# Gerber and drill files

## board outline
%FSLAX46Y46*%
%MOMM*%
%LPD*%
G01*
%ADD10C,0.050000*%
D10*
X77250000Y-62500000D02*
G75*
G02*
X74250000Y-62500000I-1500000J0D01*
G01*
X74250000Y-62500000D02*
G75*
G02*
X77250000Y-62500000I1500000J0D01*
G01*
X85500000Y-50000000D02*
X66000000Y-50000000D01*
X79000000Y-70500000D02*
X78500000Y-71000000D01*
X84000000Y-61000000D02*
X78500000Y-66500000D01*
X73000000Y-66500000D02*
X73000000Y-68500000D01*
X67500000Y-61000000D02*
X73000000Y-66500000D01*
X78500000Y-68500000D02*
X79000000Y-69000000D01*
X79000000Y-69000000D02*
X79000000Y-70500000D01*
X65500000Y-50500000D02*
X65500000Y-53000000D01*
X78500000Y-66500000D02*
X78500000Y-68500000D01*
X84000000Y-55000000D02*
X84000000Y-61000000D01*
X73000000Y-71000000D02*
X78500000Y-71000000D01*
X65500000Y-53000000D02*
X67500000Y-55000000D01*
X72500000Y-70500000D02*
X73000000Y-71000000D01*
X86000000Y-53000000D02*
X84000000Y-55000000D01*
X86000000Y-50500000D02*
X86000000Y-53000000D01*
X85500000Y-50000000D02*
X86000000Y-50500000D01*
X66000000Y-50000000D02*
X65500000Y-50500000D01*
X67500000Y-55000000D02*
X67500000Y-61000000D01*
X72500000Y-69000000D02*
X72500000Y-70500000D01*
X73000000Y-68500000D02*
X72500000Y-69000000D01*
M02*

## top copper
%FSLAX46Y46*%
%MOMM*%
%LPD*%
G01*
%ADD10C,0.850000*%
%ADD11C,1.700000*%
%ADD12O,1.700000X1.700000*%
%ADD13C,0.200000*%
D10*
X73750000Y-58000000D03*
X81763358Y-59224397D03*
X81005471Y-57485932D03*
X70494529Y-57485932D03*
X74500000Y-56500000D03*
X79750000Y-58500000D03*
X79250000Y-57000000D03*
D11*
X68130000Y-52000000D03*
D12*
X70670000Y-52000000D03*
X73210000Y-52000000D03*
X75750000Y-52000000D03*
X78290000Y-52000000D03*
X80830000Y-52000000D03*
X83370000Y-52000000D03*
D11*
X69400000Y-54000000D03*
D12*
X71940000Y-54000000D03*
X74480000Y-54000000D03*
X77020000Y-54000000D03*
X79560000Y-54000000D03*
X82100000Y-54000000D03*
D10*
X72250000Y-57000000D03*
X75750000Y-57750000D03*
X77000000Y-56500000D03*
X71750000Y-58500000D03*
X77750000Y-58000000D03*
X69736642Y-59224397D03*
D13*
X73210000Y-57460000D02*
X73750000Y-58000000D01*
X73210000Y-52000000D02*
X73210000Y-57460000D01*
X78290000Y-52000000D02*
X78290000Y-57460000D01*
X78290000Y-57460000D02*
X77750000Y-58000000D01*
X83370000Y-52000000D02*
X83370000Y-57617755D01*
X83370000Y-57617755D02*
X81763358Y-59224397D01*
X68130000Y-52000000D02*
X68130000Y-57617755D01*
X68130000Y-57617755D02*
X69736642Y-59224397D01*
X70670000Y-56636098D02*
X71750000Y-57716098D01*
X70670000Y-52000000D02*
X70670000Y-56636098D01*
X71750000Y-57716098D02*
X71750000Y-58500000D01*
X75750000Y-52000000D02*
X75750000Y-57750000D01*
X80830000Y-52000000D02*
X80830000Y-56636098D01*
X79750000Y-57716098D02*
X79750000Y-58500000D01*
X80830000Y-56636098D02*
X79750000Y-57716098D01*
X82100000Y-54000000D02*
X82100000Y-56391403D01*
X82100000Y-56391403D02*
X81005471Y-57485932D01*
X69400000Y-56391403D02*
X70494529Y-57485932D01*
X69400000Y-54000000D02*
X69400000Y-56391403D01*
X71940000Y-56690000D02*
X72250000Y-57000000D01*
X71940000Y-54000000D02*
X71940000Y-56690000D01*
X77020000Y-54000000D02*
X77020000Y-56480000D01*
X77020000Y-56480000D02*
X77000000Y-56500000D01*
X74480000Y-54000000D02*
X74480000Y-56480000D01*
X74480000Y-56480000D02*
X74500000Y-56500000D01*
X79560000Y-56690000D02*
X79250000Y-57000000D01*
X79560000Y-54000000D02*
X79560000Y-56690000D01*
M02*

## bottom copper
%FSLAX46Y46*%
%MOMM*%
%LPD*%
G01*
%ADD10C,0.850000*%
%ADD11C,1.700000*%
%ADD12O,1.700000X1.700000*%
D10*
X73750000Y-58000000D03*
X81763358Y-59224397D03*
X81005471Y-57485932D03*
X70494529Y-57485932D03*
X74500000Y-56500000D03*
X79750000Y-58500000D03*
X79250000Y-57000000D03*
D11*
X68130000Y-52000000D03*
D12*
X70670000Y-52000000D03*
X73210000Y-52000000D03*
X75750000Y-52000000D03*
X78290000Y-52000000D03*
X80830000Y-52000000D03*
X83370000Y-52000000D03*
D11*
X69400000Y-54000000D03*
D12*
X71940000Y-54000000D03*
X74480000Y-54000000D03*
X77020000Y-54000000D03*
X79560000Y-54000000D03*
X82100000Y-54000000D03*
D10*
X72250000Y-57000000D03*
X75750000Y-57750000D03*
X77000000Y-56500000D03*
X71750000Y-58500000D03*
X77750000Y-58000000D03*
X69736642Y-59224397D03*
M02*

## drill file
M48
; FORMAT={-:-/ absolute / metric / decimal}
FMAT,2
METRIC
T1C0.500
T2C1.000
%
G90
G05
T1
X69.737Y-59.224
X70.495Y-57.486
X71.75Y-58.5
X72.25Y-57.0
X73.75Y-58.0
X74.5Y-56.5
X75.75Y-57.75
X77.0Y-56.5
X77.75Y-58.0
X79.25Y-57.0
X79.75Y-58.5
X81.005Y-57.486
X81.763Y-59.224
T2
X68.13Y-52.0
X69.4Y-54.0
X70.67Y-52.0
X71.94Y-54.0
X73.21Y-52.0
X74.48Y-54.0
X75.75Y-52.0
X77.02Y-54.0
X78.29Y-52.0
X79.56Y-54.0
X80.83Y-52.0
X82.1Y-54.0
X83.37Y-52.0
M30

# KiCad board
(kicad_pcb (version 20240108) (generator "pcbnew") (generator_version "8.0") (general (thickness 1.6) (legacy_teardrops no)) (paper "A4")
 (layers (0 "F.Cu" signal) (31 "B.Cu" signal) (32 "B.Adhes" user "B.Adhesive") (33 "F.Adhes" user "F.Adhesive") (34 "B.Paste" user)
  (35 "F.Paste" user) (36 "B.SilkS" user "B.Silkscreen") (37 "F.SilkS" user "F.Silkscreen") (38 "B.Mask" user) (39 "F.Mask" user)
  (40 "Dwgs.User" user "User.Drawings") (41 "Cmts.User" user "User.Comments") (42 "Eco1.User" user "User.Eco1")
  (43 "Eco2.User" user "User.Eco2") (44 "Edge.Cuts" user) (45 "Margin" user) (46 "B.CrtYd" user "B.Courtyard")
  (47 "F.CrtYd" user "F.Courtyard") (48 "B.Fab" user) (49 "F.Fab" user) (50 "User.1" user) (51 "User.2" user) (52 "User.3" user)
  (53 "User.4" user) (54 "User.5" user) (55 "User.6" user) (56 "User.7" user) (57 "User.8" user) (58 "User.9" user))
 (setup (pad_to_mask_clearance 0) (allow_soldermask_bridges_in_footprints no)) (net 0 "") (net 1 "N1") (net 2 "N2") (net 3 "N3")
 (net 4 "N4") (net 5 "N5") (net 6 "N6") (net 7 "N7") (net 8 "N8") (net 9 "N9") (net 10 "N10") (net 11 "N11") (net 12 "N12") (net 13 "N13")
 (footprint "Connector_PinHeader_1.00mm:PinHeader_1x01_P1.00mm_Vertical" (layer "F.Cu") (at 73.75 58)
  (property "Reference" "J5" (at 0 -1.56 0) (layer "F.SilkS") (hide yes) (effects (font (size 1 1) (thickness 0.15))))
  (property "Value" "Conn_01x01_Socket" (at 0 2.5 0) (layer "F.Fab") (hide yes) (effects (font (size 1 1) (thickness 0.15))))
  (pad "1" thru_hole circle (at 0 0) (size 0.85 0.85) (drill 0.5) (layers "*.Cu" "*.Mask") (remove_unused_layers no) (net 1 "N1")))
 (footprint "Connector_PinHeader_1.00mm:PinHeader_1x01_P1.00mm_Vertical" (layer "F.Cu") (at 81.763358 59.224397)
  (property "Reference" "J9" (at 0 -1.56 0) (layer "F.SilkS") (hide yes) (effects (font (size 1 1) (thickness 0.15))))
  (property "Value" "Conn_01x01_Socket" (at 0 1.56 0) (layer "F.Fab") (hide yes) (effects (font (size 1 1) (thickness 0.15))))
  (pad "1" thru_hole circle (at 0 0) (size 0.85 0.85) (drill 0.5) (layers "*.Cu" "*.Mask") (remove_unused_layers no) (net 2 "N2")))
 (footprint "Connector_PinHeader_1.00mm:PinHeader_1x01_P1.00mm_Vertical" (layer "F.Cu") (at 81.005471 57.485932)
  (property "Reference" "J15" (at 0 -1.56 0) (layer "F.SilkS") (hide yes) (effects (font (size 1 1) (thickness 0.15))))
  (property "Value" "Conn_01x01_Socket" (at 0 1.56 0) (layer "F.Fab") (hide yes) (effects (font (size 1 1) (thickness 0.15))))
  (pad "1" thru_hole circle (at 0 0) (size 0.85 0.85) (drill 0.5) (layers "*.Cu" "*.Mask") (remove_unused_layers no) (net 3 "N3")))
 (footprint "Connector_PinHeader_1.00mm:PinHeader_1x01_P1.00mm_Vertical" (layer "F.Cu") (at 70.494529 57.485932)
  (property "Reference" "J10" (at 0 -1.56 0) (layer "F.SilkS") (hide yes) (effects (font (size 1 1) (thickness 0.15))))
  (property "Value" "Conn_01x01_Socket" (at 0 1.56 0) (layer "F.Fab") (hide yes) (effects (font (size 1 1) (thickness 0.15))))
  (pad "1" thru_hole circle (at 0 0) (size 0.85 0.85) (drill 0.5) (layers "*.Cu" "*.Mask") (remove_unused_layers no) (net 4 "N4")))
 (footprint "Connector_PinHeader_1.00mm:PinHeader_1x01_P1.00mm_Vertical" (layer "F.Cu") (at 74.5 56.5)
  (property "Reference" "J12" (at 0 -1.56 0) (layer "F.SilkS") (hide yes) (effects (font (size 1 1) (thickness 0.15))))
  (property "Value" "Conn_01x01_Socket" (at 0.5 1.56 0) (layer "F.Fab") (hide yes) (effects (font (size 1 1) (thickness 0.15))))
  (pad "1" thru_hole circle (at 0 0) (size 0.85 0.85) (drill 0.5) (layers "*.Cu" "*.Mask") (remove_unused_layers no) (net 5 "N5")))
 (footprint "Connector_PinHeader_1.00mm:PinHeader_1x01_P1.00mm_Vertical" (layer "F.Cu") (at 79.75 58.5)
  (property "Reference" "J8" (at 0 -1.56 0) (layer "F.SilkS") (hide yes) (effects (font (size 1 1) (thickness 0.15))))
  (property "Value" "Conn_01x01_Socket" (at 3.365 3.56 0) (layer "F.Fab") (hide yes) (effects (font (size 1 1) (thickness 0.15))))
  (pad "1" thru_hole circle (at 0 0) (size 0.85 0.85) (drill 0.5) (layers "*.Cu" "*.Mask") (remove_unused_layers no) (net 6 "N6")))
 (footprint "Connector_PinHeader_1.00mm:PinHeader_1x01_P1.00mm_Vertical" (layer "F.Cu") (at 79.25 57)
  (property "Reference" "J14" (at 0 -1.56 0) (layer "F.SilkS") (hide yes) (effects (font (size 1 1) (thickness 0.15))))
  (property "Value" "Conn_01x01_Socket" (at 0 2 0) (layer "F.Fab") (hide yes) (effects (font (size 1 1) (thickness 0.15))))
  (pad "1" thru_hole circle (at 0 0) (size 0.85 0.85) (drill 0.5) (layers "*.Cu" "*.Mask") (remove_unused_layers no) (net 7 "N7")))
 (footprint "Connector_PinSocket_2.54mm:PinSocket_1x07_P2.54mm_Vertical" (layer "F.Cu") (at 68.13 52 90)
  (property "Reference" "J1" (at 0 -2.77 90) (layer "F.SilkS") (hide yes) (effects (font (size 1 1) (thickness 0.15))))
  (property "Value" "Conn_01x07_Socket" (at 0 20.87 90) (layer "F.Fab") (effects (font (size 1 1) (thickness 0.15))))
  (pad "1" thru_hole circle (at 0 0 90) (size 1.7 1.7) (drill 1) (layers "*.Cu" "*.Mask") (remove_unused_layers no) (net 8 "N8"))
  (pad "2" thru_hole oval (at 0 2.54 90) (size 1.7 1.7) (drill 1) (layers "*.Cu" "*.Mask") (remove_unused_layers no) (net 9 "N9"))
  (pad "3" thru_hole oval (at 0 5.08 90) (size 1.7 1.7) (drill 1) (layers "*.Cu" "*.Mask") (remove_unused_layers no) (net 1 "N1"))
  (pad "4" thru_hole oval (at 0 7.62 90) (size 1.7 1.7) (drill 1) (layers "*.Cu" "*.Mask") (remove_unused_layers no) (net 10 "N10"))
  (pad "5" thru_hole oval (at 0 10.16 90) (size 1.7 1.7) (drill 1) (layers "*.Cu" "*.Mask") (remove_unused_layers no) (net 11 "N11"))
  (pad "6" thru_hole oval (at 0 12.7 90) (size 1.7 1.7) (drill 1) (layers "*.Cu" "*.Mask") (remove_unused_layers no) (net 6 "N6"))
  (pad "7" thru_hole oval (at 0 15.24 90) (size 1.7 1.7) (drill 1) (layers "*.Cu" "*.Mask") (remove_unused_layers no) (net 2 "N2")))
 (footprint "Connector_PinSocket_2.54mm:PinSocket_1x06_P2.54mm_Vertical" (layer "F.Cu") (at 69.4 54 90)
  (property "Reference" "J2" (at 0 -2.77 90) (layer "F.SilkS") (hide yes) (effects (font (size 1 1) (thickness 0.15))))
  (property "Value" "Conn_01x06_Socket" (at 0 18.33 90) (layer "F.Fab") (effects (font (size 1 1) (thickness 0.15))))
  (pad "1" thru_hole circle (at 0 0 90) (size 1.7 1.7) (drill 1) (layers "*.Cu" "*.Mask") (remove_unused_layers no) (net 4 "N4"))
  (pad "2" thru_hole oval (at 0 2.54 90) (size 1.7 1.7) (drill 1) (layers "*.Cu" "*.Mask") (remove_unused_layers no) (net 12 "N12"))
  (pad "3" thru_hole oval (at 0 5.08 90) (size 1.7 1.7) (drill 1) (layers "*.Cu" "*.Mask") (remove_unused_layers no) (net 5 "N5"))
  (pad "4" thru_hole oval (at 0 7.62 90) (size 1.7 1.7) (drill 1) (layers "*.Cu" "*.Mask") (remove_unused_layers no) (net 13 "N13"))
  (pad "5" thru_hole oval (at 0 10.16 90) (size 1.7 1.7) (drill 1) (layers "*.Cu" "*.Mask") (remove_unused_layers no) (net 7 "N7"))
  (pad "6" thru_hole oval (at 0 12.7 90) (size 1.7 1.7) (drill 1) (layers "*.Cu" "*.Mask") (remove_unused_layers no) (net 3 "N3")))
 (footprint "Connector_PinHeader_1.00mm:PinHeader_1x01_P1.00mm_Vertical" (layer "F.Cu") (at 72.25 57)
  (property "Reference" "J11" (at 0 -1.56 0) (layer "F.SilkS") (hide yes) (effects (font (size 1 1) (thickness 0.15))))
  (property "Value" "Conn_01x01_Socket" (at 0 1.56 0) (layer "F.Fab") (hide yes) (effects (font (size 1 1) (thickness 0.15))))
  (pad "1" thru_hole circle (at 0 0) (size 0.85 0.85) (drill 0.5) (layers "*.Cu" "*.Mask") (remove_unused_layers no) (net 12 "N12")))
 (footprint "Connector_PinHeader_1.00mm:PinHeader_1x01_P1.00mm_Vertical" (layer "F.Cu") (at 75.75 57.75)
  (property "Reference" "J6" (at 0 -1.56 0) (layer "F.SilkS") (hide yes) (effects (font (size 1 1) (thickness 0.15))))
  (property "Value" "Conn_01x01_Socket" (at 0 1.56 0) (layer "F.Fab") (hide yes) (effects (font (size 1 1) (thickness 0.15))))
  (pad "1" thru_hole circle (at 0 0) (size 0.85 0.85) (drill 0.5) (layers "*.Cu" "*.Mask") (remove_unused_layers no) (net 10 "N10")))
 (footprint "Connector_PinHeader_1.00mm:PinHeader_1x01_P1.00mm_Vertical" (layer "F.Cu") (at 77 56.5)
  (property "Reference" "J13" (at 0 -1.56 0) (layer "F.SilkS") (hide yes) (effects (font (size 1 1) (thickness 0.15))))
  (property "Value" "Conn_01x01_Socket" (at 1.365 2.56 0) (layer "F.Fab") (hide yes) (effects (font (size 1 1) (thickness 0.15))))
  (pad "1" thru_hole circle (at 0 0) (size 0.85 0.85) (drill 0.5) (layers "*.Cu" "*.Mask") (remove_unused_layers no) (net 13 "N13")))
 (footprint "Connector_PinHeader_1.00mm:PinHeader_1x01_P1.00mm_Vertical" (layer "F.Cu") (at 71.75 58.5)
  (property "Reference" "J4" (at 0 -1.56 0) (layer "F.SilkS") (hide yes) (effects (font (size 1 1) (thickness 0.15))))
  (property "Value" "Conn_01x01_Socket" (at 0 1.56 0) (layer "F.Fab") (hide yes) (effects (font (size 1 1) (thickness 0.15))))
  (pad "1" thru_hole circle (at 0 0) (size 0.85 0.85) (drill 0.5) (layers "*.Cu" "*.Mask") (remove_unused_layers no) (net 9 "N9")))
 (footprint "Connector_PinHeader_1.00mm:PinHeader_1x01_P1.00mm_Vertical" (layer "F.Cu") (at 77.75 58)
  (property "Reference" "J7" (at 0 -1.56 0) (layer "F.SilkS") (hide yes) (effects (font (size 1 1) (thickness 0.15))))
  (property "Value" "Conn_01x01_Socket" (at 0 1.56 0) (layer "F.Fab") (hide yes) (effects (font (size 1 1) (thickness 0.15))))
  (pad "1" thru_hole circle (at 0 0) (size 0.85 0.85) (drill 0.5) (layers "*.Cu" "*.Mask") (remove_unused_layers no) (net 11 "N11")))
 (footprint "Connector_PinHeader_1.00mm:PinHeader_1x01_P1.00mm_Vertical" (layer "F.Cu") (at 69.736642 59.224397)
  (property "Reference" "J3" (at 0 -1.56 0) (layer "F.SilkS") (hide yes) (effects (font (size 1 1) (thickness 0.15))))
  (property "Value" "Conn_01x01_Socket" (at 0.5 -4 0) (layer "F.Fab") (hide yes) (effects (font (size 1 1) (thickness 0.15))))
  (pad "1" thru_hole circle (at 0 0) (size 0.85 0.85) (drill 0.5) (layers "*.Cu" "*.Mask") (remove_unused_layers no) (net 8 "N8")))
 (gr_circle (center 75.75 62.5) (end 75.75 61) (stroke (width 0.05) (type default)) (fill none) (layer "Edge.Cuts"))
 (gr_line (start 85.5 50) (end 66 50) (stroke (width 0.05) (type default)) (layer "Edge.Cuts"))
 (gr_line (start 79 70.5) (end 78.5 71) (stroke (width 0.05) (type default)) (layer "Edge.Cuts"))
 (gr_line (start 84 61) (end 78.5 66.5) (stroke (width 0.05) (type default)) (layer "Edge.Cuts"))
 (gr_line (start 73 66.5) (end 73 68.5) (stroke (width 0.05) (type default)) (layer "Edge.Cuts"))
 (gr_line (start 67.5 61) (end 73 66.5) (stroke (width 0.05) (type default)) (layer "Edge.Cuts"))
 (gr_line (start 78.5 68.5) (end 79 69) (stroke (width 0.05) (type default)) (layer "Edge.Cuts"))
 (gr_line (start 79 69) (end 79 70.5) (stroke (width 0.05) (type default)) (layer "Edge.Cuts"))
 (gr_line (start 65.5 50.5) (end 65.5 53) (stroke (width 0.05) (type default)) (layer "Edge.Cuts"))
 (gr_line (start 78.5 66.5) (end 78.5 68.5) (stroke (width 0.05) (type default)) (layer "Edge.Cuts"))
 (gr_line (start 84 55) (end 84 61) (stroke (width 0.05) (type default)) (layer "Edge.Cuts"))
 (gr_line (start 73 71) (end 78.5 71) (stroke (width 0.05) (type default)) (layer "Edge.Cuts"))
 (gr_line (start 65.5 53) (end 67.5 55) (stroke (width 0.05) (type default)) (layer "Edge.Cuts"))
 (gr_line (start 72.5 70.5) (end 73 71) (stroke (width 0.05) (type default)) (layer "Edge.Cuts"))
 (gr_line (start 86 53) (end 84 55) (stroke (width 0.05) (type default)) (layer "Edge.Cuts"))
 (gr_line (start 86 50.5) (end 86 53) (stroke (width 0.05) (type default)) (layer "Edge.Cuts"))
 (gr_line (start 85.5 50) (end 86 50.5) (stroke (width 0.05) (type default)) (layer "Edge.Cuts"))
 (gr_line (start 66 50) (end 65.5 50.5) (stroke (width 0.05) (type default)) (layer "Edge.Cuts"))
 (gr_line (start 67.5 55) (end 67.5 61) (stroke (width 0.05) (type default)) (layer "Edge.Cuts"))
 (gr_line (start 72.5 69) (end 72.5 70.5) (stroke (width 0.05) (type default)) (layer "Edge.Cuts"))
 (gr_line (start 73 68.5) (end 72.5 69) (stroke (width 0.05) (type default)) (layer "Edge.Cuts"))
 (segment (start 73.21 57.46) (end 73.75 58) (width 0.2) (layer "F.Cu") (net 1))
 (segment (start 73.21 52) (end 73.21 57.46) (width 0.2) (layer "F.Cu") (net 1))
 (segment (start 78.29 52) (end 78.29 57.46) (width 0.2) (layer "F.Cu") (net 11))
 (segment (start 78.29 57.46) (end 77.75 58) (width 0.2) (layer "F.Cu") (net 11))
 (segment (start 83.37 52) (end 83.37 57.617755) (width 0.2) (layer "F.Cu") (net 2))
 (segment (start 83.37 57.617755) (end 81.763358 59.224397) (width 0.2) (layer "F.Cu") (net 2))
 (segment (start 68.13 52) (end 68.13 57.617755) (width 0.2) (layer "F.Cu") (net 8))
 (segment (start 68.13 57.617755) (end 69.736642 59.224397) (width 0.2) (layer "F.Cu") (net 8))
 (segment (start 70.67 56.636098) (end 71.75 57.716098) (width 0.2) (layer "F.Cu") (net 9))
 (segment (start 70.67 52) (end 70.67 56.636098) (width 0.2) (layer "F.Cu") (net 9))
 (segment (start 71.75 57.716098) (end 71.75 58.5) (width 0.2) (layer "F.Cu") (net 9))
 (segment (start 75.75 52) (end 75.75 57.75) (width 0.2) (layer "F.Cu") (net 10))
 (segment (start 80.83 52) (end 80.83 56.636098) (width 0.2) (layer "F.Cu") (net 6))
 (segment (start 79.75 57.716098) (end 79.75 58.5) (width 0.2) (layer "F.Cu") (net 6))
 (segment (start 80.83 56.636098) (end 79.75 57.716098) (width 0.2) (layer "F.Cu") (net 6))
 (segment (start 82.1 54) (end 82.1 56.391403) (width 0.2) (layer "F.Cu") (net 3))
 (segment (start 82.1 56.391403) (end 81.005471 57.485932) (width 0.2) (layer "F.Cu") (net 3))
 (segment (start 69.4 56.391403) (end 70.494529 57.485932) (width 0.2) (layer "F.Cu") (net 4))
 (segment (start 69.4 54) (end 69.4 56.391403) (width 0.2) (layer "F.Cu") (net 4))
 (segment (start 71.94 56.69) (end 72.25 57) (width 0.2) (layer "F.Cu") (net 12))
 (segment (start 71.94 54) (end 71.94 56.69) (width 0.2) (layer "F.Cu") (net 12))
 (segment (start 77.02 54) (end 77.02 56.48) (width 0.2) (layer "F.Cu") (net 13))
 (segment (start 77.02 56.48) (end 77 56.5) (width 0.2) (layer "F.Cu") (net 13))
 (segment (start 74.48 54) (end 74.48 56.48) (width 0.2) (layer "F.Cu") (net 5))
 (segment (start 74.48 56.48) (end 74.5 56.5) (width 0.2) (layer "F.Cu") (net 5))
 (segment (start 79.56 56.69) (end 79.25 57) (width 0.2) (layer "F.Cu") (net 7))
 (segment (start 79.56 54) (end 79.56 56.69) (width 0.2) (layer "F.Cu") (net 7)))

